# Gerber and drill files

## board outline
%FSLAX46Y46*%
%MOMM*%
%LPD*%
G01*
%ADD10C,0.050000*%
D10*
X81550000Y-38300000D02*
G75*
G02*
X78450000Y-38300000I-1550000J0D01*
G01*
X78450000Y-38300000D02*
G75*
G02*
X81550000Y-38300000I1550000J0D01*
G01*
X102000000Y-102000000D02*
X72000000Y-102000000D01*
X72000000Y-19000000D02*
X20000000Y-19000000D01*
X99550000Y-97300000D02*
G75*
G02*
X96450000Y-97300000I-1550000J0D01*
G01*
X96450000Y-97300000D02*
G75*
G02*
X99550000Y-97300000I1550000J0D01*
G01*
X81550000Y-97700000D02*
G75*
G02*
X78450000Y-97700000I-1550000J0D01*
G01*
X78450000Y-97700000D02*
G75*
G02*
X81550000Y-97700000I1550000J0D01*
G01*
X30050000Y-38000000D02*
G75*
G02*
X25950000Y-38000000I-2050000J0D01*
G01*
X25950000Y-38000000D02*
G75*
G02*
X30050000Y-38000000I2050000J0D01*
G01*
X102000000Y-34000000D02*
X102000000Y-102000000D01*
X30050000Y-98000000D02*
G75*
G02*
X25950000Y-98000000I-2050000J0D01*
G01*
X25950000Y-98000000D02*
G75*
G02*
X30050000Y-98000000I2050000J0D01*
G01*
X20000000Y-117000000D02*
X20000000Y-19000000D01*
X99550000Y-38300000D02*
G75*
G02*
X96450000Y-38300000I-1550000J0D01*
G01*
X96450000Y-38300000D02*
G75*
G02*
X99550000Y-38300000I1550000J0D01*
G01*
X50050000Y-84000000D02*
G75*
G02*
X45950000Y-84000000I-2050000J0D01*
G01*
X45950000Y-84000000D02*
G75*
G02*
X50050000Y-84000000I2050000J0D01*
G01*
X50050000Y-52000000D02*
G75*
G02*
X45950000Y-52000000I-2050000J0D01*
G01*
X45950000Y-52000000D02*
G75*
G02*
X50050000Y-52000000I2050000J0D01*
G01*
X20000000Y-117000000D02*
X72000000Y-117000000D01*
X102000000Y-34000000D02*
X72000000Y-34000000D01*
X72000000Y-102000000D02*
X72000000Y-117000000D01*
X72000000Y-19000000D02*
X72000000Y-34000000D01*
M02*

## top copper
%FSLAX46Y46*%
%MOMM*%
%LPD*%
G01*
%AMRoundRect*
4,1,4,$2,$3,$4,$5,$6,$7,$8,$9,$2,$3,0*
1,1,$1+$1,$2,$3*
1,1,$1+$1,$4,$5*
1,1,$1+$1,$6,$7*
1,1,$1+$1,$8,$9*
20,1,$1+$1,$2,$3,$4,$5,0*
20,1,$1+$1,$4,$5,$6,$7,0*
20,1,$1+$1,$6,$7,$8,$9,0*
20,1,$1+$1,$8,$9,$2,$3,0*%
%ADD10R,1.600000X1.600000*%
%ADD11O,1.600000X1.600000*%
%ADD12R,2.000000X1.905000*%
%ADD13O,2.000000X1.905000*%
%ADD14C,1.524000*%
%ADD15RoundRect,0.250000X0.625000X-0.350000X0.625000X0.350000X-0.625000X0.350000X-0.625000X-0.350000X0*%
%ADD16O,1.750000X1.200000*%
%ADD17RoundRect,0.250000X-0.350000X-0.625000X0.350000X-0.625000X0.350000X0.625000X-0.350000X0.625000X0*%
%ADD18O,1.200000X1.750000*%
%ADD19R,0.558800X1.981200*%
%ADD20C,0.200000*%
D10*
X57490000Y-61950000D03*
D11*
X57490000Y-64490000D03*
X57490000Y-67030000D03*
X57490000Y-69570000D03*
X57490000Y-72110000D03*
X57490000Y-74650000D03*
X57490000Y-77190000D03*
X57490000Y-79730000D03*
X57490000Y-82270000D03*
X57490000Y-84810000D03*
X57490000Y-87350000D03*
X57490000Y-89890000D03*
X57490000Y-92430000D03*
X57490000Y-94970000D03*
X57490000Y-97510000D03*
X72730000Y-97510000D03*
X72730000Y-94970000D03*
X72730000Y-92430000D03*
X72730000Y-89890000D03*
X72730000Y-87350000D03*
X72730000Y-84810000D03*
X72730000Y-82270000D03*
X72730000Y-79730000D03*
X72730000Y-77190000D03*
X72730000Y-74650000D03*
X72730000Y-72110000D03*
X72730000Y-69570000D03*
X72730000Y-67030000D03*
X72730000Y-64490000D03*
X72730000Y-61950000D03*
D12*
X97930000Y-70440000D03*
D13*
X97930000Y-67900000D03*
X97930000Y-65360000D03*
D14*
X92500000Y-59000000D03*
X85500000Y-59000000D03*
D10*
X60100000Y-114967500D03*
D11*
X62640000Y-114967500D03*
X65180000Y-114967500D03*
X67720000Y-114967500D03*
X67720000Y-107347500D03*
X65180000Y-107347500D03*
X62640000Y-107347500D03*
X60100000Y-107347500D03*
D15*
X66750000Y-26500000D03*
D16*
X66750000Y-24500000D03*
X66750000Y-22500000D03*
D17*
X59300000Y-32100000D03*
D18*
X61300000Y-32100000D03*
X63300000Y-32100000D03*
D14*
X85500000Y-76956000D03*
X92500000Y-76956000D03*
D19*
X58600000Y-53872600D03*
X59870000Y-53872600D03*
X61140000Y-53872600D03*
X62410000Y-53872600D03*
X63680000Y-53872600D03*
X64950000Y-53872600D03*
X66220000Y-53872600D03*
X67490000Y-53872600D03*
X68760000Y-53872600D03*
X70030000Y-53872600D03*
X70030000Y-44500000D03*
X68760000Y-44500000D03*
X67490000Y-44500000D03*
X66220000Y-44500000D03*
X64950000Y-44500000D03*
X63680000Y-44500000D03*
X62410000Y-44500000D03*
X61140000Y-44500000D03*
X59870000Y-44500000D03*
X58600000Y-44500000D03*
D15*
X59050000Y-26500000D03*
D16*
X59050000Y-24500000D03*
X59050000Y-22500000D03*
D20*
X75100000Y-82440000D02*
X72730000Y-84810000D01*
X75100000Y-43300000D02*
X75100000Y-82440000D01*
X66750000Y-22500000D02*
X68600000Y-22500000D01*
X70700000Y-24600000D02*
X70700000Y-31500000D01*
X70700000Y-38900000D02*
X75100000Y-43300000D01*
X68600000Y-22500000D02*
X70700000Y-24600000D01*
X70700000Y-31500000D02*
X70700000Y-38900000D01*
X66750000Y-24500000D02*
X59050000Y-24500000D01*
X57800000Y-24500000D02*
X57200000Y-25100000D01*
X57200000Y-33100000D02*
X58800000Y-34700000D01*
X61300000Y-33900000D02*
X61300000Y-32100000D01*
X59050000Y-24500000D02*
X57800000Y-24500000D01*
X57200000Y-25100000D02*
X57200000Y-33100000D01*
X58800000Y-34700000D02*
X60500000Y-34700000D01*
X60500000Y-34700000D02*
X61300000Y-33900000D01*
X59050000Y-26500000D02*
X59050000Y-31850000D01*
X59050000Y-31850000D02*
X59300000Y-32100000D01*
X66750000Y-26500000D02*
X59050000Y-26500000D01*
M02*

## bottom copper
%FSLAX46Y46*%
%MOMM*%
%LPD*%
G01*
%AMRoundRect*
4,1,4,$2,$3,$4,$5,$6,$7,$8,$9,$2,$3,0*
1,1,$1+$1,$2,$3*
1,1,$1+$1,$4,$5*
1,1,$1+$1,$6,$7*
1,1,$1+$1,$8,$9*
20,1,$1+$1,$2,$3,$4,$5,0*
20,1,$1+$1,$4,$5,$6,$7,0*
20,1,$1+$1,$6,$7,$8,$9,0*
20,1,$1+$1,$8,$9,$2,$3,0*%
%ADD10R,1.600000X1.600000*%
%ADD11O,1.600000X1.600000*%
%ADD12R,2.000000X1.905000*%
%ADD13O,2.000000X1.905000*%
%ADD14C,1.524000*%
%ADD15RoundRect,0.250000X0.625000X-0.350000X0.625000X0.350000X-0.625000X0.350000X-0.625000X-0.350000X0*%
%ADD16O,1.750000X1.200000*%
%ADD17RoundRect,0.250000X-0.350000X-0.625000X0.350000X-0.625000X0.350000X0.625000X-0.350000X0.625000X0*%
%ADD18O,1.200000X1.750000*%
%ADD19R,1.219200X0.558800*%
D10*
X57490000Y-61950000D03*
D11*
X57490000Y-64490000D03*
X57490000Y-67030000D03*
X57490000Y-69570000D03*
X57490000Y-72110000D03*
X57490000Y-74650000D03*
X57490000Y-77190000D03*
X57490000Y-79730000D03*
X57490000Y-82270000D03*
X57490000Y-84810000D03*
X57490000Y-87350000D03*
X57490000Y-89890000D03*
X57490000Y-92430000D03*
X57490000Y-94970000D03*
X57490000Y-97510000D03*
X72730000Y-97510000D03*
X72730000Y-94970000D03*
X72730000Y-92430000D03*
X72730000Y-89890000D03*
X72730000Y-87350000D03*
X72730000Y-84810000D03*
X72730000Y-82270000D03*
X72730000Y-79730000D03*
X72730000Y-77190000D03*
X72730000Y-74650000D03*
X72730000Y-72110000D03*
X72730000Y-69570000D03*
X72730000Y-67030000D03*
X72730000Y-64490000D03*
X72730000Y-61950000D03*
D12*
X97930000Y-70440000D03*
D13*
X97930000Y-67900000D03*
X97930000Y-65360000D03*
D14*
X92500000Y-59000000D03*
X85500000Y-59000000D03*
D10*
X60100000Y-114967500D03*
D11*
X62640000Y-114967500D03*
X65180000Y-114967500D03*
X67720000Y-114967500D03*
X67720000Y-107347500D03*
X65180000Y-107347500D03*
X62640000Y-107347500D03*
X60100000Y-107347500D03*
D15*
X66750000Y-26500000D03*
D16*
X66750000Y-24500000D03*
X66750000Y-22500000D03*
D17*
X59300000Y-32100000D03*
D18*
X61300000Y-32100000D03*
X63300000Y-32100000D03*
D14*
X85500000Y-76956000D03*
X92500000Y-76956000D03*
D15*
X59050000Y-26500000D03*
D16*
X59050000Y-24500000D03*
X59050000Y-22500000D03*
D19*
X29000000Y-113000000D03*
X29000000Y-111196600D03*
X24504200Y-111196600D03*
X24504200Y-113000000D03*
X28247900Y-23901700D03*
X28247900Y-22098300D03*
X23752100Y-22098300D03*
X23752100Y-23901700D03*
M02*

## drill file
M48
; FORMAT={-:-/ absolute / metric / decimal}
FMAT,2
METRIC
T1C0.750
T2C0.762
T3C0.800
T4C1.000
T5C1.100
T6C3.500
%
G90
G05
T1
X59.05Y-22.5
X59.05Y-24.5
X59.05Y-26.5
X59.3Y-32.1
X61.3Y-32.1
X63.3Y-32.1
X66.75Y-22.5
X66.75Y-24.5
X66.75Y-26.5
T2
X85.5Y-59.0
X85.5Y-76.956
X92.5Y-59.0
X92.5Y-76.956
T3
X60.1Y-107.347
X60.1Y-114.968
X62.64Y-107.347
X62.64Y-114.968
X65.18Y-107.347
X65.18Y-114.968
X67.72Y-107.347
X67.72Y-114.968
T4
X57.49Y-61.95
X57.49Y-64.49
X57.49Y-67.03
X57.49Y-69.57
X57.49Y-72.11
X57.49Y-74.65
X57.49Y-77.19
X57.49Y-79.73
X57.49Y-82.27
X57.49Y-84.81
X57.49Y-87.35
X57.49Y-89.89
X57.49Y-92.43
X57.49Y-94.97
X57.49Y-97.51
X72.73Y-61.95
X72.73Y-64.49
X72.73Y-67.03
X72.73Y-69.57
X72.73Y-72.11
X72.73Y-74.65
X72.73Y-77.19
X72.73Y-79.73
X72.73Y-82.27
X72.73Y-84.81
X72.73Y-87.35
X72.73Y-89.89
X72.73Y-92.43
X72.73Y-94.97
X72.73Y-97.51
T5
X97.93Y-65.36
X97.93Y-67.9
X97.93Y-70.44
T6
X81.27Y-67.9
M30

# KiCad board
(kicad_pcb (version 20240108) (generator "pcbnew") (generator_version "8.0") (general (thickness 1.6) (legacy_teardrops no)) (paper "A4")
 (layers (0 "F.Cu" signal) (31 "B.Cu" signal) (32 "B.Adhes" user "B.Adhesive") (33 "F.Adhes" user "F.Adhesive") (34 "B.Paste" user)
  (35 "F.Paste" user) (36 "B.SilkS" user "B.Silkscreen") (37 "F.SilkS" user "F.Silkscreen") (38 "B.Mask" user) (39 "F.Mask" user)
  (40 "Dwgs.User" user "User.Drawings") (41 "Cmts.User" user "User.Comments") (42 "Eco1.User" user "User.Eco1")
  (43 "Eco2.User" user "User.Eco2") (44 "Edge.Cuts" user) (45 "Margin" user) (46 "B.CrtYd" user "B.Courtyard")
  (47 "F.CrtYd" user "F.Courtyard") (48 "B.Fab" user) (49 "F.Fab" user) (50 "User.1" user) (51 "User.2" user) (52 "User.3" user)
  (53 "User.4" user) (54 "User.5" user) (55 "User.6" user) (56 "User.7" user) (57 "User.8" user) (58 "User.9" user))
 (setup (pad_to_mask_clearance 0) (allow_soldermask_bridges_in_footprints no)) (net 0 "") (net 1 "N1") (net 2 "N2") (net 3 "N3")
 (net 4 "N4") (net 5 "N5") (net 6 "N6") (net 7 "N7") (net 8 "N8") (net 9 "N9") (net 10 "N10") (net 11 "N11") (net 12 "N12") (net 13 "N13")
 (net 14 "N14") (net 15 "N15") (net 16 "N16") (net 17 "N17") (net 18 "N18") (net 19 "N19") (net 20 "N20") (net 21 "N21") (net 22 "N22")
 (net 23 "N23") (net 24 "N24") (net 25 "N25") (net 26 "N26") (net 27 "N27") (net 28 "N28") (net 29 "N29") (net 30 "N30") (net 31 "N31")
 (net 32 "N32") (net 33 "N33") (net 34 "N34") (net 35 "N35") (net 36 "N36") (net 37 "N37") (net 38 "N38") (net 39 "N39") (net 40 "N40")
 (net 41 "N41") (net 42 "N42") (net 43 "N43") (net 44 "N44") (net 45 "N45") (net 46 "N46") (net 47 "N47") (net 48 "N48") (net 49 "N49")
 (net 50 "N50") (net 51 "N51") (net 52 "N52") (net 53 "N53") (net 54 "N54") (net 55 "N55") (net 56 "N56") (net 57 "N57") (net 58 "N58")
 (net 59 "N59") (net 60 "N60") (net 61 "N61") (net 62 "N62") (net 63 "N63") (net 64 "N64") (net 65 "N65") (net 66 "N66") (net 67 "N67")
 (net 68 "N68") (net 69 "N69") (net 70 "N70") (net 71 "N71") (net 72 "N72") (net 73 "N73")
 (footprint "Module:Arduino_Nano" (layer "F.Cu") (at 57.49 61.95)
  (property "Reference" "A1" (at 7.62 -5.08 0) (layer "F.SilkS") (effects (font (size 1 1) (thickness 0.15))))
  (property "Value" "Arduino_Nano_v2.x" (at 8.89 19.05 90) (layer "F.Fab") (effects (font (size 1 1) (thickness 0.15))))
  (pad "1" thru_hole rect (at 0 0) (size 1.6 1.6) (drill 1) (layers "*.Cu" "*.Mask") (remove_unused_layers no) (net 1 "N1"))
  (pad "2" thru_hole oval (at 0 2.54) (size 1.6 1.6) (drill 1) (layers "*.Cu" "*.Mask") (remove_unused_layers no) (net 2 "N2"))
  (pad "3" thru_hole oval (at 0 5.08) (size 1.6 1.6) (drill 1) (layers "*.Cu" "*.Mask") (remove_unused_layers no) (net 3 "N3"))
  (pad "4" thru_hole oval (at 0 7.62) (size 1.6 1.6) (drill 1) (layers "*.Cu" "*.Mask") (remove_unused_layers no) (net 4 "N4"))
  (pad "5" thru_hole oval (at 0 10.16) (size 1.6 1.6) (drill 1) (layers "*.Cu" "*.Mask") (remove_unused_layers no) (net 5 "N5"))
  (pad "6" thru_hole oval (at 0 12.7) (size 1.6 1.6) (drill 1) (layers "*.Cu" "*.Mask") (remove_unused_layers no) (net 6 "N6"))
  (pad "7" thru_hole oval (at 0 15.24) (size 1.6 1.6) (drill 1) (layers "*.Cu" "*.Mask") (remove_unused_layers no) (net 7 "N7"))
  (pad "8" thru_hole oval (at 0 17.78) (size 1.6 1.6) (drill 1) (layers "*.Cu" "*.Mask") (remove_unused_layers no) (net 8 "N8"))
  (pad "9" thru_hole oval (at 0 20.32) (size 1.6 1.6) (drill 1) (layers "*.Cu" "*.Mask") (remove_unused_layers no) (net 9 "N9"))
  (pad "10" thru_hole oval (at 0 22.86) (size 1.6 1.6) (drill 1) (layers "*.Cu" "*.Mask") (remove_unused_layers no) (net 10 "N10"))
  (pad "11" thru_hole oval (at 0 25.4) (size 1.6 1.6) (drill 1) (layers "*.Cu" "*.Mask") (remove_unused_layers no) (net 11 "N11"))
  (pad "12" thru_hole oval (at 0 27.94) (size 1.6 1.6) (drill 1) (layers "*.Cu" "*.Mask") (remove_unused_layers no) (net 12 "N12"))
  (pad "13" thru_hole oval (at 0 30.48) (size 1.6 1.6) (drill 1) (layers "*.Cu" "*.Mask") (remove_unused_layers no) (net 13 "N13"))
  (pad "14" thru_hole oval (at 0 33.02) (size 1.6 1.6) (drill 1) (layers "*.Cu" "*.Mask") (remove_unused_layers no) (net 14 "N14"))
  (pad "15" thru_hole oval (at 0 35.56) (size 1.6 1.6) (drill 1) (layers "*.Cu" "*.Mask") (remove_unused_layers no) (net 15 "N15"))
  (pad "16" thru_hole oval (at 15.24 35.56) (size 1.6 1.6) (drill 1) (layers "*.Cu" "*.Mask") (remove_unused_layers no) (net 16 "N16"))
  (pad "17" thru_hole oval (at 15.24 33.02) (size 1.6 1.6) (drill 1) (layers "*.Cu" "*.Mask") (remove_unused_layers no) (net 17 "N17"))
  (pad "18" thru_hole oval (at 15.24 30.48) (size 1.6 1.6) (drill 1) (layers "*.Cu" "*.Mask") (remove_unused_layers no) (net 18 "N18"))
  (pad "19" thru_hole oval (at 15.24 27.94) (size 1.6 1.6) (drill 1) (layers "*.Cu" "*.Mask") (remove_unused_layers no) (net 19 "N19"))
  (pad "20" thru_hole oval (at 15.24 25.4) (size 1.6 1.6) (drill 1) (layers "*.Cu" "*.Mask") (remove_unused_layers no) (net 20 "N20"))
  (pad "21" thru_hole oval (at 15.24 22.86) (size 1.6 1.6) (drill 1) (layers "*.Cu" "*.Mask") (remove_unused_layers no) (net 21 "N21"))
  (pad "22" thru_hole oval (at 15.24 20.32) (size 1.6 1.6) (drill 1) (layers "*.Cu" "*.Mask") (remove_unused_layers no) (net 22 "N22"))
  (pad "23" thru_hole oval (at 15.24 17.78) (size 1.6 1.6) (drill 1) (layers "*.Cu" "*.Mask") (remove_unused_layers no) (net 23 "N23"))
  (pad "24" thru_hole oval (at 15.24 15.24) (size 1.6 1.6) (drill 1) (layers "*.Cu" "*.Mask") (remove_unused_layers no) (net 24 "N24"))
  (pad "25" thru_hole oval (at 15.24 12.7) (size 1.6 1.6) (drill 1) (layers "*.Cu" "*.Mask") (remove_unused_layers no) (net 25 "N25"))
  (pad "26" thru_hole oval (at 15.24 10.16) (size 1.6 1.6) (drill 1) (layers "*.Cu" "*.Mask") (remove_unused_layers no) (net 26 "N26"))
  (pad "27" thru_hole oval (at 15.24 7.62) (size 1.6 1.6) (drill 1) (layers "*.Cu" "*.Mask") (remove_unused_layers no) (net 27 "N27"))
  (pad "28" thru_hole oval (at 15.24 5.08) (size 1.6 1.6) (drill 1) (layers "*.Cu" "*.Mask") (remove_unused_layers no) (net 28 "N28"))
  (pad "29" thru_hole oval (at 15.24 2.54) (size 1.6 1.6) (drill 1) (layers "*.Cu" "*.Mask") (remove_unused_layers no) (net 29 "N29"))
  (pad "30" thru_hole oval (at 15.24 0) (size 1.6 1.6) (drill 1) (layers "*.Cu" "*.Mask") (remove_unused_layers no) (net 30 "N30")))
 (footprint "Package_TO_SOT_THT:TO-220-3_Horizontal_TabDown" (layer "F.Cu") (at 97.93 70.44 90)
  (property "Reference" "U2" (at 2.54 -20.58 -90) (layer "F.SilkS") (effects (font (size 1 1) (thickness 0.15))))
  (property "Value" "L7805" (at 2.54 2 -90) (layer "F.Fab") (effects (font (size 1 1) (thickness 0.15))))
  (pad "" np_thru_hole oval (at 2.54 -16.66 90) (size 3.5 3.5) (drill 3.5) (layers "*.Cu" "*.Mask"))
  (pad "1" thru_hole rect (at 0 0 90) (size 1.905 2) (drill 1.1) (layers "*.Cu" "*.Mask") (remove_unused_layers no) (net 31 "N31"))
  (pad "2" thru_hole oval (at 2.54 0 90) (size 1.905 2) (drill 1.1) (layers "*.Cu" "*.Mask") (remove_unused_layers no) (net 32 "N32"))
  (pad "3" thru_hole oval (at 5.08 0 90) (size 1.905 2) (drill 1.1) (layers "*.Cu" "*.Mask") (remove_unused_layers no) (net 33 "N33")))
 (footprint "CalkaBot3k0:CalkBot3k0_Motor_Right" (layer "F.Cu") (at 102 34 180)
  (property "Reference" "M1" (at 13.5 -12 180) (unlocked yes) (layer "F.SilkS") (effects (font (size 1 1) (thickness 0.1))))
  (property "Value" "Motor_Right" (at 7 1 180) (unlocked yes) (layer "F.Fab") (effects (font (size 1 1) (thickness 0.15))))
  (pad "1" thru_hole circle (at 9.5 -25 180) (size 1.524 1.524) (drill 0.762) (layers "*.Cu" "*.Mask") (remove_unused_layers no)
   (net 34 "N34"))
  (pad "2" thru_hole circle (at 16.5 -25 180) (size 1.524 1.524) (drill 0.762) (layers "*.Cu" "*.Mask") (remove_unused_layers no)
   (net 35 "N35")))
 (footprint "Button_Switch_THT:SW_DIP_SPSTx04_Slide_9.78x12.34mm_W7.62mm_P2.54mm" (layer "F.Cu") (at 60.1 114.9675 90)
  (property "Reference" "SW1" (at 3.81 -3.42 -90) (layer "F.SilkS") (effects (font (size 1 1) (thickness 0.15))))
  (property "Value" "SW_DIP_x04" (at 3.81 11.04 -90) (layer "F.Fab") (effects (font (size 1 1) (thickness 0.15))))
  (pad "1" thru_hole rect (at 0 0 90) (size 1.6 1.6) (drill 0.8) (layers "*.Cu" "*.Mask") (remove_unused_layers no) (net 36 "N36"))
  (pad "2" thru_hole oval (at 0 2.54 90) (size 1.6 1.6) (drill 0.8) (layers "*.Cu" "*.Mask") (remove_unused_layers no) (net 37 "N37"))
  (pad "3" thru_hole oval (at 0 5.08 90) (size 1.6 1.6) (drill 0.8) (layers "*.Cu" "*.Mask") (remove_unused_layers no) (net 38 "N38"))
  (pad "4" thru_hole oval (at 0 7.62 90) (size 1.6 1.6) (drill 0.8) (layers "*.Cu" "*.Mask") (remove_unused_layers no) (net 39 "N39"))
  (pad "5" thru_hole oval (at 7.62 7.62 90) (size 1.6 1.6) (drill 0.8) (layers "*.Cu" "*.Mask") (remove_unused_layers no) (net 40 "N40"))
  (pad "6" thru_hole oval (at 7.62 5.08 90) (size 1.6 1.6) (drill 0.8) (layers "*.Cu" "*.Mask") (remove_unused_layers no) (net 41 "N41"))
  (pad "7" thru_hole oval (at 7.62 2.54 90) (size 1.6 1.6) (drill 0.8) (layers "*.Cu" "*.Mask") (remove_unused_layers no) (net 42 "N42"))
  (pad "8" thru_hole oval (at 7.62 0 90) (size 1.6 1.6) (drill 0.8) (layers "*.Cu" "*.Mask") (remove_unused_layers no) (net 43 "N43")))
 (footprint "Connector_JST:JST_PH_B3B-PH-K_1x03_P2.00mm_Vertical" (layer "F.Cu") (at 66.75 26.5 90)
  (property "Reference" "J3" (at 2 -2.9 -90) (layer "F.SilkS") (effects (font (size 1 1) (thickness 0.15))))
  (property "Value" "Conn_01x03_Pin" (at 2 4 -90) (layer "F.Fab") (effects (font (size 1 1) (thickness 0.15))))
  (pad "1" thru_hole roundrect (at 0 0 90) (size 1.2 1.75) (drill 0.75) (layers "*.Cu" "*.Mask") (remove_unused_layers no)
   (roundrect_rratio 0.208333) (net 30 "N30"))
  (pad "2" thru_hole oval (at 2 0 90) (size 1.2 1.75) (drill 0.75) (layers "*.Cu" "*.Mask") (remove_unused_layers no) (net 4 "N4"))
  (pad "3" thru_hole oval (at 4 0 90) (size 1.2 1.75) (drill 0.75) (layers "*.Cu" "*.Mask") (remove_unused_layers no) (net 21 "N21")))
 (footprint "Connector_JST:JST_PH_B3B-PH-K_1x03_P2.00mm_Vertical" (layer "F.Cu") (at 59.3 32.1)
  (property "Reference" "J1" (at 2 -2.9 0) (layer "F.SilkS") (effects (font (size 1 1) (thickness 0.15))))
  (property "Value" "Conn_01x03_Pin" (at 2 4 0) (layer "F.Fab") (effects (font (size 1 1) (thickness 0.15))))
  (pad "1" thru_hole roundrect (at 0 0) (size 1.2 1.75) (drill 0.75) (layers "*.Cu" "*.Mask") (remove_unused_layers no)
   (roundrect_rratio 0.208333) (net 30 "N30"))
  (pad "2" thru_hole oval (at 2 0) (size 1.2 1.75) (drill 0.75) (layers "*.Cu" "*.Mask") (remove_unused_layers no) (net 4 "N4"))
  (pad "3" thru_hole oval (at 4 0) (size 1.2 1.75) (drill 0.75) (layers "*.Cu" "*.Mask") (remove_unused_layers no) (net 19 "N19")))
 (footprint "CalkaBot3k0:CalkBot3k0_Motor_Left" (layer "F.Cu") (at 76 101.956)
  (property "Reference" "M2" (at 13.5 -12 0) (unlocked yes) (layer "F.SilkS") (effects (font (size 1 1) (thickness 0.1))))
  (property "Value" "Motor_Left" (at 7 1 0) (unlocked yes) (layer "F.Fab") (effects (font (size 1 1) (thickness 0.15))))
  (pad "1" thru_hole circle (at 9.5 -25) (size 1.524 1.524) (drill 0.762) (layers "*.Cu" "*.Mask") (remove_unused_layers no) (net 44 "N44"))
  (pad "2" thru_hole circle (at 16.5 -25) (size 1.524 1.524) (drill 0.762) (layers "*.Cu" "*.Mask") (remove_unused_layers no) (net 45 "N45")))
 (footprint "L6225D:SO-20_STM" (layer "F.Cu") (at 64.315 49.1863 90)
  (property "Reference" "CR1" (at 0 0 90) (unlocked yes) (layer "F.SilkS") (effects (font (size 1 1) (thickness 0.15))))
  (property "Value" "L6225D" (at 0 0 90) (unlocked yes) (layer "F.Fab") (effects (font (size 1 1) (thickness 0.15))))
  (pad "1" smd rect (at -4.6863 -5.715 90) (size 1.9812 0.5588) (layers "F.Cu" "F.Paste" "F.Mask") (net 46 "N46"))
  (pad "2" smd rect (at -4.6863 -4.445 90) (size 1.9812 0.5588) (layers "F.Cu" "F.Paste" "F.Mask") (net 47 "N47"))
  (pad "3" smd rect (at -4.6863 -3.175 90) (size 1.9812 0.5588) (layers "F.Cu" "F.Paste" "F.Mask") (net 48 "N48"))
  (pad "4" smd rect (at -4.6863 -1.905 90) (size 1.9812 0.5588) (layers "F.Cu" "F.Paste" "F.Mask") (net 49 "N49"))
  (pad "5" smd rect (at -4.6863 -0.635 90) (size 1.9812 0.5588) (layers "F.Cu" "F.Paste" "F.Mask") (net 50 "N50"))
  (pad "6" smd rect (at -4.6863 0.635 90) (size 1.9812 0.5588) (layers "F.Cu" "F.Paste" "F.Mask") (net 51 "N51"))
  (pad "7" smd rect (at -4.6863 1.905 90) (size 1.9812 0.5588) (layers "F.Cu" "F.Paste" "F.Mask") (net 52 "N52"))
  (pad "8" smd rect (at -4.6863 3.175 90) (size 1.9812 0.5588) (layers "F.Cu" "F.Paste" "F.Mask") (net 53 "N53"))
  (pad "9" smd rect (at -4.6863 4.445 90) (size 1.9812 0.5588) (layers "F.Cu" "F.Paste" "F.Mask") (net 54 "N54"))
  (pad "10" smd rect (at -4.6863 5.715 90) (size 1.9812 0.5588) (layers "F.Cu" "F.Paste" "F.Mask") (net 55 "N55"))
  (pad "11" smd rect (at 4.6863 5.715 90) (size 1.9812 0.5588) (layers "F.Cu" "F.Paste" "F.Mask") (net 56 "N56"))
  (pad "12" smd rect (at 4.6863 4.445 90) (size 1.9812 0.5588) (layers "F.Cu" "F.Paste" "F.Mask") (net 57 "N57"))
  (pad "13" smd rect (at 4.6863 3.175 90) (size 1.9812 0.5588) (layers "F.Cu" "F.Paste" "F.Mask") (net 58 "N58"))
  (pad "14" smd rect (at 4.6863 1.905 90) (size 1.9812 0.5588) (layers "F.Cu" "F.Paste" "F.Mask") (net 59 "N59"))
  (pad "15" smd rect (at 4.6863 0.635 90) (size 1.9812 0.5588) (layers "F.Cu" "F.Paste" "F.Mask") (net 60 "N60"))
  (pad "16" smd rect (at 4.6863 -0.635 90) (size 1.9812 0.5588) (layers "F.Cu" "F.Paste" "F.Mask") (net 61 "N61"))
  (pad "17" smd rect (at 4.6863 -1.905 90) (size 1.9812 0.5588) (layers "F.Cu" "F.Paste" "F.Mask") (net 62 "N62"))
  (pad "18" smd rect (at 4.6863 -3.175 90) (size 1.9812 0.5588) (layers "F.Cu" "F.Paste" "F.Mask") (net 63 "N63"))
  (pad "19" smd rect (at 4.6863 -4.445 90) (size 1.9812 0.5588) (layers "F.Cu" "F.Paste" "F.Mask") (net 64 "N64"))
  (pad "20" smd rect (at 4.6863 -5.715 90) (size 1.9812 0.5588) (layers "F.Cu" "F.Paste" "F.Mask") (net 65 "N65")))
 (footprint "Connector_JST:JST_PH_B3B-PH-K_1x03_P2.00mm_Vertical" (layer "F.Cu") (at 59.05 26.5 90)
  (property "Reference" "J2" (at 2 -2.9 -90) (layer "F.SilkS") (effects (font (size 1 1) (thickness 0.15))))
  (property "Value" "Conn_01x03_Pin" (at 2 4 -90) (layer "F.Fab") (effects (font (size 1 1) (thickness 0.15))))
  (pad "1" thru_hole roundrect (at 0 0 90) (size 1.2 1.75) (drill 0.75) (layers "*.Cu" "*.Mask") (remove_unused_layers no)
   (roundrect_rratio 0.208333) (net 30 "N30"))
  (pad "2" thru_hole oval (at 2 0 90) (size 1.2 1.75) (drill 0.75) (layers "*.Cu" "*.Mask") (remove_unused_layers no) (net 4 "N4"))
  (pad "3" thru_hole oval (at 4 0 90) (size 1.2 1.75) (drill 0.75) (layers "*.Cu" "*.Mask") (remove_unused_layers no) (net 20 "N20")))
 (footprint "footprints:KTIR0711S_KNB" (layer "B.Cu") (at 26.7521 112.0983 180)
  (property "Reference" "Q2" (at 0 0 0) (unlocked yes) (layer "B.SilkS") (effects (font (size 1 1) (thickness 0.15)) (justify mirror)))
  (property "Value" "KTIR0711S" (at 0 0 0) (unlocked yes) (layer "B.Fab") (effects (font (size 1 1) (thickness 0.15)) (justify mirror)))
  (pad "1" smd rect (at -2.2479 -0.9017 180) (size 1.2192 0.5588) (layers "B.Cu" "B.Paste" "B.Mask") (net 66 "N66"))
  (pad "2" smd rect (at -2.2479 0.9017 180) (size 1.2192 0.5588) (layers "B.Cu" "B.Paste" "B.Mask") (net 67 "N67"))
  (pad "3" smd rect (at 2.2479 0.9017 180) (size 1.2192 0.5588) (layers "B.Cu" "B.Paste" "B.Mask") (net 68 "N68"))
  (pad "4" smd rect (at 2.2479 -0.9017 180) (size 1.2192 0.5588) (layers "B.Cu" "B.Paste" "B.Mask") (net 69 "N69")))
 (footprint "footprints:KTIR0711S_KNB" (layer "B.Cu") (at 26 23 180)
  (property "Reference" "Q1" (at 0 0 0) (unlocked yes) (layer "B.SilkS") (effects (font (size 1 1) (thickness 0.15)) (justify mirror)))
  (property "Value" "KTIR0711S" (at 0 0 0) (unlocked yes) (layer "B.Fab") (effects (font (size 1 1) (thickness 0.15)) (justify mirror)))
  (pad "1" smd rect (at -2.2479 -0.9017 180) (size 1.2192 0.5588) (layers "B.Cu" "B.Paste" "B.Mask") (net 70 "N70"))
  (pad "2" smd rect (at -2.2479 0.9017 180) (size 1.2192 0.5588) (layers "B.Cu" "B.Paste" "B.Mask") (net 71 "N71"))
  (pad "3" smd rect (at 2.2479 0.9017 180) (size 1.2192 0.5588) (layers "B.Cu" "B.Paste" "B.Mask") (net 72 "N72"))
  (pad "4" smd rect (at 2.2479 -0.9017 180) (size 1.2192 0.5588) (layers "B.Cu" "B.Paste" "B.Mask") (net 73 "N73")))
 (gr_circle (center 80 38.3) (end 81.55 38.3) (stroke (width 0.05) (type default)) (fill none) (layer "Edge.Cuts"))
 (gr_line (start 102 102) (end 72 102) (stroke (width 0.05) (type default)) (layer "Edge.Cuts"))
 (gr_line (start 72 19) (end 20 19) (stroke (width 0.05) (type default)) (layer "Edge.Cuts"))
 (gr_circle (center 98 97.3) (end 99.55 97.3) (stroke (width 0.05) (type default)) (fill none) (layer "Edge.Cuts"))
 (gr_circle (center 80 97.7) (end 81.55 97.7) (stroke (width 0.05) (type default)) (fill none) (layer "Edge.Cuts"))
 (gr_circle (center 28 38) (end 30.05 38) (stroke (width 0.05) (type default)) (fill none) (layer "Edge.Cuts"))
 (gr_line (start 102 34) (end 102 102) (stroke (width 0.05) (type default)) (layer "Edge.Cuts"))
 (gr_circle (center 28 98) (end 30.05 98) (stroke (width 0.05) (type default)) (fill none) (layer "Edge.Cuts"))
 (gr_line (start 20 117) (end 20 19) (stroke (width 0.05) (type default)) (layer "Edge.Cuts"))
 (gr_circle (center 98 38.3) (end 99.55 38.3) (stroke (width 0.05) (type default)) (fill none) (layer "Edge.Cuts"))
 (gr_circle (center 48 84) (end 50.05 84) (stroke (width 0.05) (type default)) (fill none) (layer "Edge.Cuts"))
 (gr_circle (center 48 52) (end 50.05 52) (stroke (width 0.05) (type default)) (fill none) (layer "Edge.Cuts"))
 (gr_line (start 20 117) (end 72 117) (stroke (width 0.05) (type default)) (layer "Edge.Cuts"))
 (gr_line (start 102 34) (end 72 34) (stroke (width 0.05) (type default)) (layer "Edge.Cuts"))
 (gr_line (start 72 102) (end 72 117) (stroke (width 0.05) (type default)) (layer "Edge.Cuts"))
 (gr_line (start 72 19) (end 72 34) (stroke (width 0.05) (type default)) (layer "Edge.Cuts"))
 (segment (start 75.1 82.44) (end 72.73 84.81) (width 0.2) (layer "F.Cu") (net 21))
 (segment (start 75.1 43.3) (end 75.1 82.44) (width 0.2) (layer "F.Cu") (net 21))
 (segment (start 66.75 22.5) (end 68.6 22.5) (width 0.2) (layer "F.Cu") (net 21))
 (segment (start 70.7 24.6) (end 70.7 31.5) (width 0.2) (layer "F.Cu") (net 21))
 (segment (start 70.7 38.9) (end 75.1 43.3) (width 0.2) (layer "F.Cu") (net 21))
 (segment (start 68.6 22.5) (end 70.7 24.6) (width 0.2) (layer "F.Cu") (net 21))
 (segment (start 70.7 31.5) (end 70.7 38.9) (width 0.2) (layer "F.Cu") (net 21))
 (segment (start 66.75 24.5) (end 59.05 24.5) (width 0.2) (layer "F.Cu") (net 4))
 (segment (start 57.8 24.5) (end 57.2 25.1) (width 0.2) (layer "F.Cu") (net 4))
 (segment (start 57.2 33.1) (end 58.8 34.7) (width 0.2) (layer "F.Cu") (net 4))
 (segment (start 61.3 33.9) (end 61.3 32.1) (width 0.2) (layer "F.Cu") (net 4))
 (segment (start 59.05 24.5) (end 57.8 24.5) (width 0.2) (layer "F.Cu") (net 4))
 (segment (start 57.2 25.1) (end 57.2 33.1) (width 0.2) (layer "F.Cu") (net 4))
 (segment (start 58.8 34.7) (end 60.5 34.7) (width 0.2) (layer "F.Cu") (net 4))
 (segment (start 60.5 34.7) (end 61.3 33.9) (width 0.2) (layer "F.Cu") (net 4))
 (segment (start 59.05 26.5) (end 59.05 31.85) (width 0.2) (layer "F.Cu") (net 30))
 (segment (start 59.05 31.85) (end 59.3 32.1) (width 0.2) (layer "F.Cu") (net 30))
 (segment (start 66.75 26.5) (end 59.05 26.5) (width 0.2) (layer "F.Cu") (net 30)))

